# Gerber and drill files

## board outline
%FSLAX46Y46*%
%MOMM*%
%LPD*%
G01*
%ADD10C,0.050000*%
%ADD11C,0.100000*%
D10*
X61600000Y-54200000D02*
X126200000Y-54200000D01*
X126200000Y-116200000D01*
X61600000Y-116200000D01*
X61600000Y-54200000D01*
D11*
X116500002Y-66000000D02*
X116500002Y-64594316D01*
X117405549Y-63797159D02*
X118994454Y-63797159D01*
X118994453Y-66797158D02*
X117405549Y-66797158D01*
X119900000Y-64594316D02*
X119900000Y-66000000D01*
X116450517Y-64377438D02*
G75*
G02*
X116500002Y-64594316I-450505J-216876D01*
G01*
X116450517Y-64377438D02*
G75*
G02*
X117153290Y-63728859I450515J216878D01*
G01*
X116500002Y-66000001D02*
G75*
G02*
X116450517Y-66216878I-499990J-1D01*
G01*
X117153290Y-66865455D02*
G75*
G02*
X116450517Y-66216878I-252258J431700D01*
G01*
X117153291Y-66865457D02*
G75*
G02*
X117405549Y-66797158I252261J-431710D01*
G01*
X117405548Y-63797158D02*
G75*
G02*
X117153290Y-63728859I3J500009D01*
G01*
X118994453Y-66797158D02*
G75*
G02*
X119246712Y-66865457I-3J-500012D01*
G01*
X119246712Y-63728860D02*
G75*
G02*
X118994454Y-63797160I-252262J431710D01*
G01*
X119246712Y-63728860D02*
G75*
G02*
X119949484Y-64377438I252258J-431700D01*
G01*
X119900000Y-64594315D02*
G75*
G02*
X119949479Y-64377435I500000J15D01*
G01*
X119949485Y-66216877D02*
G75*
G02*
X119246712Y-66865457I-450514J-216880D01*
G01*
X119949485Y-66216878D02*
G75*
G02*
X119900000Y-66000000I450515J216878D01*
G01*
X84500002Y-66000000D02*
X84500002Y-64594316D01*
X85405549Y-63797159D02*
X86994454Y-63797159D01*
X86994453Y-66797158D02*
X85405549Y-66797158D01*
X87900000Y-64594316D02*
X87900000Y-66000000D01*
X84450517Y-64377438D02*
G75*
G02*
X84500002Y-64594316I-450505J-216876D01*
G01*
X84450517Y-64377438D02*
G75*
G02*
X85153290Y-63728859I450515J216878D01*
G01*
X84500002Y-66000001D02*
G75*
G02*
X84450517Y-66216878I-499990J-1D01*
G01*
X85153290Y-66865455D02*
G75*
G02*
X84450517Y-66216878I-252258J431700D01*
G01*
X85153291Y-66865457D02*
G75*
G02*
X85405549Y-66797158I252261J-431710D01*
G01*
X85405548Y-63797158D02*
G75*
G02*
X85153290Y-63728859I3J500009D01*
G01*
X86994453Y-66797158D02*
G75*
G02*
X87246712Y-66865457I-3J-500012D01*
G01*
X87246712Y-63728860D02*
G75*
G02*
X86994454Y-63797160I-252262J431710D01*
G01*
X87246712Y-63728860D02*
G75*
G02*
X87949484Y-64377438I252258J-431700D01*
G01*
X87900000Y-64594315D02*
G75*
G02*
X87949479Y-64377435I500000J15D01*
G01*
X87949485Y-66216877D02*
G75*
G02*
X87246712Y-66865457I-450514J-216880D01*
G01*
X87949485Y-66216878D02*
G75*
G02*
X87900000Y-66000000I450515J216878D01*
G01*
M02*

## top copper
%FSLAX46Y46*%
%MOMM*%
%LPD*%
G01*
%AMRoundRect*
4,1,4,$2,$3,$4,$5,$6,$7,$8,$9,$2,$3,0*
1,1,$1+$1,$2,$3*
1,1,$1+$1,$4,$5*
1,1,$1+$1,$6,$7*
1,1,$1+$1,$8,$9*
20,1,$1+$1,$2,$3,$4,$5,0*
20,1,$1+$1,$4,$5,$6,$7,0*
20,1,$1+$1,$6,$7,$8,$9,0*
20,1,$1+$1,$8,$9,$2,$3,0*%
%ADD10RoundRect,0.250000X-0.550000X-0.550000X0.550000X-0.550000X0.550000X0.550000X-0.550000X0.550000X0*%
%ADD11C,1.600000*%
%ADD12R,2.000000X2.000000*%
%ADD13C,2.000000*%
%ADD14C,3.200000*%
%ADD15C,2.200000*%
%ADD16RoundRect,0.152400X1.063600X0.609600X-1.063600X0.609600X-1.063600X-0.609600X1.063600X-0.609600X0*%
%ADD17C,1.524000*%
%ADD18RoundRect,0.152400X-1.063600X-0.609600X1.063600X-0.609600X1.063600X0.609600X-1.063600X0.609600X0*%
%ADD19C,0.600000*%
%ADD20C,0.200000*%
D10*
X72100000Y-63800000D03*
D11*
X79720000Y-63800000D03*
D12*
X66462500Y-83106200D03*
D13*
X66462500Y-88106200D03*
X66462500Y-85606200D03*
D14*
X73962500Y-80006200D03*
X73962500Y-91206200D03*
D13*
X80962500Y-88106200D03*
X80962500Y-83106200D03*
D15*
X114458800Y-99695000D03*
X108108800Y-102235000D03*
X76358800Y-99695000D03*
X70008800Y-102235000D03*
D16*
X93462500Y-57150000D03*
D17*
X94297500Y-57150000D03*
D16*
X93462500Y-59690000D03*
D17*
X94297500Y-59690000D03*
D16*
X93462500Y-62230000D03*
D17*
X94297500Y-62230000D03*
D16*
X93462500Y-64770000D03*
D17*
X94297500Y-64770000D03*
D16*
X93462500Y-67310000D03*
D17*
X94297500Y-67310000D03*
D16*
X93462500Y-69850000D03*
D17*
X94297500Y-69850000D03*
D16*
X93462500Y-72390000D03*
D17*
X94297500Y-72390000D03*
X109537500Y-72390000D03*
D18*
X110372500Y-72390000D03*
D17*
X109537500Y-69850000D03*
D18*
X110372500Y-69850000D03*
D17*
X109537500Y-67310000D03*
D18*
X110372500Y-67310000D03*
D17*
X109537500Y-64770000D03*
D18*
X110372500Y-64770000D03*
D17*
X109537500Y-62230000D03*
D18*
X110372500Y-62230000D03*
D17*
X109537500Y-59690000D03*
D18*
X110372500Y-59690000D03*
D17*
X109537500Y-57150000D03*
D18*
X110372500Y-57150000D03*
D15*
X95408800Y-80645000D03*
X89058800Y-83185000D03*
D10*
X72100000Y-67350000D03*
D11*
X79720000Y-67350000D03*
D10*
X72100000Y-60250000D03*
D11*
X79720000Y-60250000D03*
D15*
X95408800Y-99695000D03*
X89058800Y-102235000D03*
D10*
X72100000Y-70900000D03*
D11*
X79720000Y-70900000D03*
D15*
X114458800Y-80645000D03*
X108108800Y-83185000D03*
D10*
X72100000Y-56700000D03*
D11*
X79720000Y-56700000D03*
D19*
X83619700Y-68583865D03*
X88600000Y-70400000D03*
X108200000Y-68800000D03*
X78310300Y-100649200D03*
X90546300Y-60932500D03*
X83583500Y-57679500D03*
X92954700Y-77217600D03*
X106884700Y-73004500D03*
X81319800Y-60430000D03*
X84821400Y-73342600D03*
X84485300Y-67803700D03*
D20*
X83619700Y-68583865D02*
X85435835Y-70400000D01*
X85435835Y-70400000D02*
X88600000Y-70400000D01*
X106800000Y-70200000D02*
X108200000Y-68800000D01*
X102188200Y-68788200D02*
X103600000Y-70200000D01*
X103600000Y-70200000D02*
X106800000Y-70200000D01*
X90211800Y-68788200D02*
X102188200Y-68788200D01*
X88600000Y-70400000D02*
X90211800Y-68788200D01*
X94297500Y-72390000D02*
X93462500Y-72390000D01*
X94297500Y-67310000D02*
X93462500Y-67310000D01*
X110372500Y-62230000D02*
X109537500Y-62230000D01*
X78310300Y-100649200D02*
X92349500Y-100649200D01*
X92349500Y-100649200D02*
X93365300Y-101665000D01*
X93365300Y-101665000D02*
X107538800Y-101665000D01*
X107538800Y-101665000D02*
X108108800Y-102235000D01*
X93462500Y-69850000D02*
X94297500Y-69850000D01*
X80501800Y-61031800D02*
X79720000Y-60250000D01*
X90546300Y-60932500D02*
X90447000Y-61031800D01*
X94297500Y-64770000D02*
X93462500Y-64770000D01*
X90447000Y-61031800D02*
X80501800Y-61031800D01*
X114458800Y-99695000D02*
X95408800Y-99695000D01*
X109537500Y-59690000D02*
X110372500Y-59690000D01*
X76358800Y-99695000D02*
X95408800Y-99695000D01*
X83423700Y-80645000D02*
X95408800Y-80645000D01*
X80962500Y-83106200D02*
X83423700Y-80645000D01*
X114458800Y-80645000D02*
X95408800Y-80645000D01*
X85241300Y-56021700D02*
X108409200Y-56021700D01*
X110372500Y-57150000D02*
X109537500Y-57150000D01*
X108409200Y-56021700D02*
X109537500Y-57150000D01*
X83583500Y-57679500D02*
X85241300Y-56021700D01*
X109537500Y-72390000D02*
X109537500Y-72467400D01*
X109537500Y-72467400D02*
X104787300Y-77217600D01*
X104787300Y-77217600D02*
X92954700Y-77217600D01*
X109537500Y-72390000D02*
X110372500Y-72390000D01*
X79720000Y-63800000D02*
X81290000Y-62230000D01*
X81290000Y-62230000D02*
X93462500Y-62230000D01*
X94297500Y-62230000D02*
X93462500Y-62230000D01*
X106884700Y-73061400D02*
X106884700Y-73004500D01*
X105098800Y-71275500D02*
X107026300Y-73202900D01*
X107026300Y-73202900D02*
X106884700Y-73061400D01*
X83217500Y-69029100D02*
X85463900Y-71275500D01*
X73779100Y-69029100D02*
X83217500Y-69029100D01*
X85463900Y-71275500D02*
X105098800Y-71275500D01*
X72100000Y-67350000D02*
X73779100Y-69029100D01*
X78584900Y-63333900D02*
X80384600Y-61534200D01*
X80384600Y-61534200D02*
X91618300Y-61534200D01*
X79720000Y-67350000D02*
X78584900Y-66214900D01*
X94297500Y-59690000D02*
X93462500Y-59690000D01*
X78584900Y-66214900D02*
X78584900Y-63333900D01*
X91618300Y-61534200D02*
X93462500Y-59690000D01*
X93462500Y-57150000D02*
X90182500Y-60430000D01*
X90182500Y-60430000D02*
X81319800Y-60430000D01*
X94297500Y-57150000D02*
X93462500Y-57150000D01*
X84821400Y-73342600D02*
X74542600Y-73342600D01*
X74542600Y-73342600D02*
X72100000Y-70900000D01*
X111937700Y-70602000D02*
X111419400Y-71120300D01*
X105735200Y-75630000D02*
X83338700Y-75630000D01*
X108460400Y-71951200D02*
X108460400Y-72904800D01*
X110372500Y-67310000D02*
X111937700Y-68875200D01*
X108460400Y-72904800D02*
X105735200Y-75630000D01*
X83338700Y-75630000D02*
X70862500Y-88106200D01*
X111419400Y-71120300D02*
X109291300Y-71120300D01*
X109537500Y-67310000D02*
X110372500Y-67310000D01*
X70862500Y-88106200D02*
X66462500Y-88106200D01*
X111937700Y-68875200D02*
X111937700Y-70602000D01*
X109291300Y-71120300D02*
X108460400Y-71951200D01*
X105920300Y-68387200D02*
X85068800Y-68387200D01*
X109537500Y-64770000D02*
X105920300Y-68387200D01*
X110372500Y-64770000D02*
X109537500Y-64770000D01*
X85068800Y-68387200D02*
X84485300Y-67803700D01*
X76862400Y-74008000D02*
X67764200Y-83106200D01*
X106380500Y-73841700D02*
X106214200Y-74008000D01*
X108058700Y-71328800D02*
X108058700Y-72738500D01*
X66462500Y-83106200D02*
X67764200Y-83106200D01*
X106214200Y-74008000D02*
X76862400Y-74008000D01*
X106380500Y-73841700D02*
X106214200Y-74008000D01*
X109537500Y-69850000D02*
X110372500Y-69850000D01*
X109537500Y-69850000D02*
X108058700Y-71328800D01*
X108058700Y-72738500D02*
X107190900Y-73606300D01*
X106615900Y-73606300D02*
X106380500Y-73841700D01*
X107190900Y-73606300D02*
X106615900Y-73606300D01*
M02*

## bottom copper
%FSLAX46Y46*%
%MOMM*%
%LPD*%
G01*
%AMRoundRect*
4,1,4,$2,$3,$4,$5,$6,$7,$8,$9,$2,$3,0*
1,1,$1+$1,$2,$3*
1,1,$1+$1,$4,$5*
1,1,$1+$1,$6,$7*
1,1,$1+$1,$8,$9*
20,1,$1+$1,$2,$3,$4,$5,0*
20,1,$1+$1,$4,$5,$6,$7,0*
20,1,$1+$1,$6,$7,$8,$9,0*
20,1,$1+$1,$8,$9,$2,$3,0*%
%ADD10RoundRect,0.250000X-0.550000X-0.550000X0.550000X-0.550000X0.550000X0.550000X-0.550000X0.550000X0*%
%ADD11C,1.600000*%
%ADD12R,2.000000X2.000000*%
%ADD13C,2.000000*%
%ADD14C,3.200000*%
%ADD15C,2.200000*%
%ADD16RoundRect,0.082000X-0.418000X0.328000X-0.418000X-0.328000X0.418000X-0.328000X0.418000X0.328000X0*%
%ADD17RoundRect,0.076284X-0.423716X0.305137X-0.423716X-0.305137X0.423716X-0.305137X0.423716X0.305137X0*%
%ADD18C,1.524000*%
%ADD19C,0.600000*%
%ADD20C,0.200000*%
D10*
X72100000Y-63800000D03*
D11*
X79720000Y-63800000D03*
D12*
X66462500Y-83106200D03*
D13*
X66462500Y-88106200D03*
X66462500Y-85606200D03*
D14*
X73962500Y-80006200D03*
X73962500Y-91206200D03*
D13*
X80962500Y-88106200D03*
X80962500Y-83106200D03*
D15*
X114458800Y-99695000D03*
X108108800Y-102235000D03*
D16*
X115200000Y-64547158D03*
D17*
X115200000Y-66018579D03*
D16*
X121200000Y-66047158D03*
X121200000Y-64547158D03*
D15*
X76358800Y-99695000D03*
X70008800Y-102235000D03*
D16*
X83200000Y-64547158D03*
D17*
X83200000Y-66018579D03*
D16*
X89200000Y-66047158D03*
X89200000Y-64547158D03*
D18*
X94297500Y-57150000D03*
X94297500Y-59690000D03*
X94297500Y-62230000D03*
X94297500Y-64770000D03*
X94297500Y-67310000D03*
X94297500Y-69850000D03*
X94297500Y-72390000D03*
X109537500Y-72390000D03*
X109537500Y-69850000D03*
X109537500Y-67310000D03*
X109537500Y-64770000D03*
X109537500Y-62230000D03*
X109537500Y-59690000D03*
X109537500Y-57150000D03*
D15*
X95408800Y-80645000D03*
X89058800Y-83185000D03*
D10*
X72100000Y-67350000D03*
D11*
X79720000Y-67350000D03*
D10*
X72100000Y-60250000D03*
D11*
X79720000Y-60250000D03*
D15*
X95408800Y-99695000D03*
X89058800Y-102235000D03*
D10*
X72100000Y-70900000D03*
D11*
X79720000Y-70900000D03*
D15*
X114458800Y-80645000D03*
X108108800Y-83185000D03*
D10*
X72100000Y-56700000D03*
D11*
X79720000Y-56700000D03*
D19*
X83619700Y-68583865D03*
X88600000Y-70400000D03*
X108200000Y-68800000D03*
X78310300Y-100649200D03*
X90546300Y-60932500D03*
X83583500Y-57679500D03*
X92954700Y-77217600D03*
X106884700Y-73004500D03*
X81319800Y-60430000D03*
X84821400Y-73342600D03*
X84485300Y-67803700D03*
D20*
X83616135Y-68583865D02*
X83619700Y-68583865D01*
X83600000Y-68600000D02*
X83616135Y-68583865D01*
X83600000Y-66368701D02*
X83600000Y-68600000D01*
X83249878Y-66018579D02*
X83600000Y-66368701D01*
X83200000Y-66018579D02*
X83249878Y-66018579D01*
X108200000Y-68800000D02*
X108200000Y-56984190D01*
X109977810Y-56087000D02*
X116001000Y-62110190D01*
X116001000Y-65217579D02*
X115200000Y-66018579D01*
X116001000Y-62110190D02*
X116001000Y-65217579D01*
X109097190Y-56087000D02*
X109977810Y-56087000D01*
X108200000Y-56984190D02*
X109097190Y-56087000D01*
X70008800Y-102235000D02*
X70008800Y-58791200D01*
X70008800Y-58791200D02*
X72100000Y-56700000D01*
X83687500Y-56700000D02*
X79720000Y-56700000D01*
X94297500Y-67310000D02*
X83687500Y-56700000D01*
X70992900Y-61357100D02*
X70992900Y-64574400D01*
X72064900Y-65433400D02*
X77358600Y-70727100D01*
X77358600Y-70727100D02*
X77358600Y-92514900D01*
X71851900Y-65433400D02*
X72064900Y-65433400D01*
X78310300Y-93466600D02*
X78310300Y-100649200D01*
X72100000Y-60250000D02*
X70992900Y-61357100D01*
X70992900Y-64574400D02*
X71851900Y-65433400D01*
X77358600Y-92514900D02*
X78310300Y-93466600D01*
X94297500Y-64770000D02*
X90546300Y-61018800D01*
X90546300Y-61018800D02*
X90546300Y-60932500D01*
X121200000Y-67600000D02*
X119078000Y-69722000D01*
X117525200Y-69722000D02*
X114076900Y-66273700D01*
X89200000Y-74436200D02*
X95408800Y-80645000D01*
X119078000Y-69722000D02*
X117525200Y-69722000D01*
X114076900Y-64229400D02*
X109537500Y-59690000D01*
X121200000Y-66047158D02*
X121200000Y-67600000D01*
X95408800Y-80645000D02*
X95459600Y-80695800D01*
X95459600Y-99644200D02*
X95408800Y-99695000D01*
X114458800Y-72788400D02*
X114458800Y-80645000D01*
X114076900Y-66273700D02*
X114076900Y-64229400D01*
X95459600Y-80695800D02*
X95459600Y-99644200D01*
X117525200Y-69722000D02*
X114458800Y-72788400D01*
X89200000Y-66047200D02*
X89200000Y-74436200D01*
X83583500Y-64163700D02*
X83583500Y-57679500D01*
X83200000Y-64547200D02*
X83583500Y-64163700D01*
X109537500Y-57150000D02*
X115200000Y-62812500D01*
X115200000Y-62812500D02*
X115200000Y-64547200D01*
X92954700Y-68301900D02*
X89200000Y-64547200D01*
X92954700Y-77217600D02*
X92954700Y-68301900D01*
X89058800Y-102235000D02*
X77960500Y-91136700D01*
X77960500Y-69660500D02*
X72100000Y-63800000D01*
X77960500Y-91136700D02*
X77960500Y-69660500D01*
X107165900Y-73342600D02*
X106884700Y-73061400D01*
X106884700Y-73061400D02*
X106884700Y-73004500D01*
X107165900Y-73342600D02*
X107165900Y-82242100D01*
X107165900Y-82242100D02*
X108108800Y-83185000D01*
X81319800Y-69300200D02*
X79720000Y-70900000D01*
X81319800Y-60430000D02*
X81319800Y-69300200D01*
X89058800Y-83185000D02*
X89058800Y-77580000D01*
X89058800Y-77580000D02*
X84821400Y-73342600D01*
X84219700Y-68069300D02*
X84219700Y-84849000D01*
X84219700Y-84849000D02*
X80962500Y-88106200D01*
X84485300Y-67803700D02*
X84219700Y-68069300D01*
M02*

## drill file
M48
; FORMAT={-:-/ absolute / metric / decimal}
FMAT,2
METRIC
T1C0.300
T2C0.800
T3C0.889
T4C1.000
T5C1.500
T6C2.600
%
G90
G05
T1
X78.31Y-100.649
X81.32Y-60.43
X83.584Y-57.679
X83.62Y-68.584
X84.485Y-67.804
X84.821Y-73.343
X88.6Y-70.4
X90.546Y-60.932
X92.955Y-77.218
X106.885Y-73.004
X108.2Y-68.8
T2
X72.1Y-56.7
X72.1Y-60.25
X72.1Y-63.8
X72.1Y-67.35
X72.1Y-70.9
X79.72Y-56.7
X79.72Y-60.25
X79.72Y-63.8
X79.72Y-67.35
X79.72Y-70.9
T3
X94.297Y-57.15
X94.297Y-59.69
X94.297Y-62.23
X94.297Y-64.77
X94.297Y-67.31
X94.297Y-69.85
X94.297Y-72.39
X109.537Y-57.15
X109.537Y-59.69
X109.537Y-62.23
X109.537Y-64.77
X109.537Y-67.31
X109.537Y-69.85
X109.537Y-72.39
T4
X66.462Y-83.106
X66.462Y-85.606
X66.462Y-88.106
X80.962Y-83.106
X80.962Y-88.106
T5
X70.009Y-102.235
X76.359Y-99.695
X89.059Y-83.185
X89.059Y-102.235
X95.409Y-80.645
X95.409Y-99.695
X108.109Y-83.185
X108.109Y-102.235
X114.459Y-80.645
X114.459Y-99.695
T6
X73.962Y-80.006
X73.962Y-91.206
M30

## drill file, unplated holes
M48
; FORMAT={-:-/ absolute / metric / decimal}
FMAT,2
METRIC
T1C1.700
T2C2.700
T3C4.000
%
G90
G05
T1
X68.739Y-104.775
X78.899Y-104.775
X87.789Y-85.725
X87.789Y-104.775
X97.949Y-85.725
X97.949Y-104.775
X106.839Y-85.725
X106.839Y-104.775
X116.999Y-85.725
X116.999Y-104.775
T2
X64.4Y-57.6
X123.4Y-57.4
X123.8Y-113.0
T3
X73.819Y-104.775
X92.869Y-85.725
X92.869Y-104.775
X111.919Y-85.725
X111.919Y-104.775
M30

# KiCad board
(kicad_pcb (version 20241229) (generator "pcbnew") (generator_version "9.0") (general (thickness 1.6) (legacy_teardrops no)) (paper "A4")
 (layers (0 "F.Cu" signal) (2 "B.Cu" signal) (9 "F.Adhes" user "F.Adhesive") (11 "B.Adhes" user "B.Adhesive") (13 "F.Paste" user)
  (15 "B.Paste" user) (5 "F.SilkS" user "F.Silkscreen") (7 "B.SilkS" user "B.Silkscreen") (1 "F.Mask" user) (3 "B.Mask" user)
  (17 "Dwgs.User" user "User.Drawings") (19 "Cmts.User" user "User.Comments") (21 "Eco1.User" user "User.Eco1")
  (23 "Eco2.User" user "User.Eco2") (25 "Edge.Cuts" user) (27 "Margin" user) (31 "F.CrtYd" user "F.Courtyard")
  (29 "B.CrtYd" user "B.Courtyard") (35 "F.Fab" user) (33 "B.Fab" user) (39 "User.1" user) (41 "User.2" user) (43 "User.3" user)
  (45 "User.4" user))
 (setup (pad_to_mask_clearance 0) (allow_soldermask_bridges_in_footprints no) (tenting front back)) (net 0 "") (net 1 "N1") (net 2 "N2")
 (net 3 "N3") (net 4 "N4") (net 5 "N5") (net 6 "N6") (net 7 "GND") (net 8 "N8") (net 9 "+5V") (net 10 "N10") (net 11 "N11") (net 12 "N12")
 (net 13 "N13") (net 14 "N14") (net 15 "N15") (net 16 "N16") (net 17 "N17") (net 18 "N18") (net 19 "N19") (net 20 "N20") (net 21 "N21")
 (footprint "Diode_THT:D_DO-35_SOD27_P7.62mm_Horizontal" (layer "F.Cu") (at 72.1 63.8)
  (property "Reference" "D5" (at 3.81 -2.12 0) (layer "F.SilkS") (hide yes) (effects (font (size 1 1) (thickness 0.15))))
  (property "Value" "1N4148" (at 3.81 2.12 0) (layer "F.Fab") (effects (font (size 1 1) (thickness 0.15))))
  (pad "1" thru_hole roundrect (at 0 0) (size 1.6 1.6) (drill 0.8) (layers "*.Cu" "*.Mask") (remove_unused_layers no)
   (roundrect_rratio 0.15625) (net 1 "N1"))
  (pad "2" thru_hole circle (at 7.62 0) (size 1.6 1.6) (drill 0.8) (layers "*.Cu" "*.Mask") (remove_unused_layers no) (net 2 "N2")))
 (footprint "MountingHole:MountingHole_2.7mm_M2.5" (layer "F.Cu") (at 123.4 57.4)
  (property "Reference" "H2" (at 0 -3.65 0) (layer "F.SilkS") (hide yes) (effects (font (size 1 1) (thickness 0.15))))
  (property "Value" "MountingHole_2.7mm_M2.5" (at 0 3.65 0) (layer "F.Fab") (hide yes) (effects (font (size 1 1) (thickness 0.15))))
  (pad "" np_thru_hole circle (at 0 0) (size 2.7 2.7) (drill 2.7) (layers "*.Cu" "*.Mask")))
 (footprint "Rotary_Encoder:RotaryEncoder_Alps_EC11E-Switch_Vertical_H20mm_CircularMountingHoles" (layer "F.Cu") (at 66.4625 83.1062)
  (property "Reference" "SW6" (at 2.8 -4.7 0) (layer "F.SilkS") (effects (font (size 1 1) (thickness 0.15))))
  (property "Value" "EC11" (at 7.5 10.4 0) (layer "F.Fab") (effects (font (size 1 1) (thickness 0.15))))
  (pad "A" thru_hole rect (at 0 0) (size 2 2) (drill 1) (layers "*.Cu" "*.Mask") (remove_unused_layers no) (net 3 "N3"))
  (pad "B" thru_hole circle (at 0 5) (size 2 2) (drill 1) (layers "*.Cu" "*.Mask") (remove_unused_layers no) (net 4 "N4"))
  (pad "C" thru_hole circle (at 0 2.5) (size 2 2) (drill 1) (layers "*.Cu" "*.Mask") (remove_unused_layers no) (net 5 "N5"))
  (pad "MP" thru_hole circle (at 7.5 -3.1) (size 3.2 3.2) (drill 2.6) (layers "*.Cu" "*.Mask") (remove_unused_layers no))
  (pad "MP" thru_hole circle (at 7.5 8.1) (size 3.2 3.2) (drill 2.6) (layers "*.Cu" "*.Mask") (remove_unused_layers no))
  (pad "S1" thru_hole circle (at 14.5 5) (size 2 2) (drill 1) (layers "*.Cu" "*.Mask") (remove_unused_layers no) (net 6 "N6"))
  (pad "S2" thru_hole circle (at 14.5 0) (size 2 2) (drill 1) (layers "*.Cu" "*.Mask") (remove_unused_layers no) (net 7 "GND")))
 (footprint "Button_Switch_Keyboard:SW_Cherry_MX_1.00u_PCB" (layer "F.Cu") (at 114.4588 99.695)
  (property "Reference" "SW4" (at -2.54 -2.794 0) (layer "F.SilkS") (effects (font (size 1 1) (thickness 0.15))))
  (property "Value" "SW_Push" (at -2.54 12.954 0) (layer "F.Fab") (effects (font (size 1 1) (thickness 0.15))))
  (pad "" np_thru_hole circle (at -7.62 5.08) (size 1.7 1.7) (drill 1.7) (layers "*.Cu" "*.Mask"))
  (pad "" np_thru_hole circle (at -2.54 5.08) (size 4 4) (drill 4) (layers "*.Cu" "*.Mask"))
  (pad "" np_thru_hole circle (at 2.54 5.08) (size 1.7 1.7) (drill 1.7) (layers "*.Cu" "*.Mask"))
  (pad "1" thru_hole circle (at 0 0) (size 2.2 2.2) (drill 1.5) (layers "*.Cu" "*.Mask") (remove_unused_layers no) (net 7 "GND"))
  (pad "2" thru_hole circle (at -6.35 2.54) (size 2.2 2.2) (drill 1.5) (layers "*.Cu" "*.Mask") (remove_unused_layers no) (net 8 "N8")))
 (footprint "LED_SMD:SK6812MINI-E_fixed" (layer "F.Cu") (at 118.2 65.4)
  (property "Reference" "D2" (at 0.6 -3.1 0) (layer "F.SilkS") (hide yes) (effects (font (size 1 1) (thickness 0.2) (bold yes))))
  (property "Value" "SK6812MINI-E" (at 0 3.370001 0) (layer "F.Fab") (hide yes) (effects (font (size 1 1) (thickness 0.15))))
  (fp_line (start -1.699998 0.6) (end -1.699998 -0.805684) (stroke (width 0.1) (type solid)) (layer "Edge.Cuts"))
  (fp_line (start -0.794451 -1.602841) (end 0.794454 -1.602841) (stroke (width 0.1) (type solid)) (layer "Edge.Cuts"))
  (fp_line (start 0.794453 1.397158) (end -0.794451 1.397158) (stroke (width 0.1) (type solid)) (layer "Edge.Cuts"))
  (fp_line (start 1.7 -0.805684) (end 1.7 0.6) (stroke (width 0.1) (type solid)) (layer "Edge.Cuts"))
  (fp_arc (start -1.749483 -1.022562) (mid -1.712526 -0.91691) (end -1.699998 -0.805684) (stroke (width 0.1) (type solid))
   (layer "Edge.Cuts"))
  (fp_arc (start -1.749483 -1.022562) (mid -1.63807 -1.606877) (end -1.04671 -1.671141) (stroke (width 0.1) (type solid))
   (layer "Edge.Cuts"))
  (fp_arc (start -1.699998 0.600001) (mid -1.712526 0.711226) (end -1.749483 0.816878) (stroke (width 0.1) (type solid)) (layer "Edge.Cuts"))
  (fp_arc (start -1.04671 1.465455) (mid -1.638069 1.401192) (end -1.749483 0.816878) (stroke (width 0.1) (type solid)) (layer "Edge.Cuts"))
  (fp_arc (start -1.046709 1.465457) (mid -0.925121 1.414535) (end -0.794451 1.397158) (stroke (width 0.1) (type solid)) (layer "Edge.Cuts"))
  (fp_arc (start -0.794452 -1.602842) (mid -0.925122 -1.620219) (end -1.04671 -1.671141) (stroke (width 0.1) (type solid))
   (layer "Edge.Cuts"))
  (fp_arc (start 0.794453 1.397158) (mid 0.925124 1.414535) (end 1.046712 1.465457) (stroke (width 0.1) (type solid)) (layer "Edge.Cuts"))
  (fp_arc (start 1.046712 -1.67114) (mid 0.925124 -1.620218) (end 0.794454 -1.602841) (stroke (width 0.1) (type solid)) (layer "Edge.Cuts"))
  (fp_arc (start 1.046712 -1.67114) (mid 1.638072 -1.606876) (end 1.749485 -1.022562) (stroke (width 0.1) (type solid)) (layer "Edge.Cuts"))
  (fp_arc (start 1.7 -0.805685) (mid 1.712528 -0.91691) (end 1.749485 -1.022562) (stroke (width 0.1) (type solid)) (layer "Edge.Cuts"))
  (fp_arc (start 1.749485 0.816877) (mid 1.638073 1.401193) (end 1.046712 1.465457) (stroke (width 0.1) (type solid)) (layer "Edge.Cuts"))
  (fp_arc (start 1.749485 0.816878) (mid 1.712528 0.711226) (end 1.7 0.6) (stroke (width 0.1) (type solid)) (layer "Edge.Cuts"))
  (pad "1" smd roundrect (at -3 -0.852842 270) (size 0.82 1) (layers "B.Cu" "B.Mask" "B.Paste") (roundrect_rratio 0.1) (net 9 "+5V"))
  (pad "2" smd roundrect (at -3 0.618579 270) (size 0.762842 1) (layers "B.Cu" "B.Mask" "B.Paste") (roundrect_rratio 0.1))
  (pad "3" smd roundrect (at 3 0.647158 270) (size 0.82 1) (layers "B.Cu" "B.Mask" "B.Paste") (roundrect_rratio 0.1) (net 7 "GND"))
  (pad "4" smd roundrect (at 3 -0.852842 270) (size 0.82 1) (layers "B.Cu" "B.Mask" "B.Paste") (roundrect_rratio 0.1) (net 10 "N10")))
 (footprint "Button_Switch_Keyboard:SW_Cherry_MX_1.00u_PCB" (layer "F.Cu") (at 76.3588 99.695)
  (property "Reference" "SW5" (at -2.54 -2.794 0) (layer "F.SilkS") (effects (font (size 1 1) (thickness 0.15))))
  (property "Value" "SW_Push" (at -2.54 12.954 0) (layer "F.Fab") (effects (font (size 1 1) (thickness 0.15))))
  (pad "" np_thru_hole circle (at -7.62 5.08) (size 1.7 1.7) (drill 1.7) (layers "*.Cu" "*.Mask"))
  (pad "" np_thru_hole circle (at -2.54 5.08) (size 4 4) (drill 4) (layers "*.Cu" "*.Mask"))
  (pad "" np_thru_hole circle (at 2.54 5.08) (size 1.7 1.7) (drill 1.7) (layers "*.Cu" "*.Mask"))
  (pad "1" thru_hole circle (at 0 0) (size 2.2 2.2) (drill 1.5) (layers "*.Cu" "*.Mask") (remove_unused_layers no) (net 7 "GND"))
  (pad "2" thru_hole circle (at -6.35 2.54) (size 2.2 2.2) (drill 1.5) (layers "*.Cu" "*.Mask") (remove_unused_layers no) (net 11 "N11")))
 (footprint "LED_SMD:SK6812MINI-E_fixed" (layer "F.Cu") (at 86.2 65.4)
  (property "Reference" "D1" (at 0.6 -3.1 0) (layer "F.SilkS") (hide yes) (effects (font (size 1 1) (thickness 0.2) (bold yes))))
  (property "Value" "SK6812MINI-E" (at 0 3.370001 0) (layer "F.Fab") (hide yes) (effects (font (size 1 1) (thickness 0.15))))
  (fp_line (start -1.699998 0.6) (end -1.699998 -0.805684) (stroke (width 0.1) (type solid)) (layer "Edge.Cuts"))
  (fp_line (start -0.794451 -1.602841) (end 0.794454 -1.602841) (stroke (width 0.1) (type solid)) (layer "Edge.Cuts"))
  (fp_line (start 0.794453 1.397158) (end -0.794451 1.397158) (stroke (width 0.1) (type solid)) (layer "Edge.Cuts"))
  (fp_line (start 1.7 -0.805684) (end 1.7 0.6) (stroke (width 0.1) (type solid)) (layer "Edge.Cuts"))
  (fp_arc (start -1.749483 -1.022562) (mid -1.712526 -0.91691) (end -1.699998 -0.805684) (stroke (width 0.1) (type solid))
   (layer "Edge.Cuts"))
  (fp_arc (start -1.749483 -1.022562) (mid -1.63807 -1.606877) (end -1.04671 -1.671141) (stroke (width 0.1) (type solid))
   (layer "Edge.Cuts"))
  (fp_arc (start -1.699998 0.600001) (mid -1.712526 0.711226) (end -1.749483 0.816878) (stroke (width 0.1) (type solid)) (layer "Edge.Cuts"))
  (fp_arc (start -1.04671 1.465455) (mid -1.638069 1.401192) (end -1.749483 0.816878) (stroke (width 0.1) (type solid)) (layer "Edge.Cuts"))
  (fp_arc (start -1.046709 1.465457) (mid -0.925121 1.414535) (end -0.794451 1.397158) (stroke (width 0.1) (type solid)) (layer "Edge.Cuts"))
  (fp_arc (start -0.794452 -1.602842) (mid -0.925122 -1.620219) (end -1.04671 -1.671141) (stroke (width 0.1) (type solid))
   (layer "Edge.Cuts"))
  (fp_arc (start 0.794453 1.397158) (mid 0.925124 1.414535) (end 1.046712 1.465457) (stroke (width 0.1) (type solid)) (layer "Edge.Cuts"))
  (fp_arc (start 1.046712 -1.67114) (mid 0.925124 -1.620218) (end 0.794454 -1.602841) (stroke (width 0.1) (type solid)) (layer "Edge.Cuts"))
  (fp_arc (start 1.046712 -1.67114) (mid 1.638072 -1.606876) (end 1.749485 -1.022562) (stroke (width 0.1) (type solid)) (layer "Edge.Cuts"))
  (fp_arc (start 1.7 -0.805685) (mid 1.712528 -0.91691) (end 1.749485 -1.022562) (stroke (width 0.1) (type solid)) (layer "Edge.Cuts"))
  (fp_arc (start 1.749485 0.816877) (mid 1.638073 1.401193) (end 1.046712 1.465457) (stroke (width 0.1) (type solid)) (layer "Edge.Cuts"))
  (fp_arc (start 1.749485 0.816878) (mid 1.712528 0.711226) (end 1.7 0.6) (stroke (width 0.1) (type solid)) (layer "Edge.Cuts"))
  (pad "1" smd roundrect (at -3 -0.852842 270) (size 0.82 1) (layers "B.Cu" "B.Mask" "B.Paste") (roundrect_rratio 0.1) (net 9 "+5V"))
  (pad "2" smd roundrect (at -3 0.618579 270) (size 0.762842 1) (layers "B.Cu" "B.Mask" "B.Paste") (roundrect_rratio 0.1))
  (pad "3" smd roundrect (at 3 0.647158 270) (size 0.82 1) (layers "B.Cu" "B.Mask" "B.Paste") (roundrect_rratio 0.1) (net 7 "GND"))
  (pad "4" smd roundrect (at 3 -0.852842 270) (size 0.82 1) (layers "B.Cu" "B.Mask" "B.Paste") (roundrect_rratio 0.1) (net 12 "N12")))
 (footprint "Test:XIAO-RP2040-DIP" (layer "F.Cu") (at 101.9175 64.77)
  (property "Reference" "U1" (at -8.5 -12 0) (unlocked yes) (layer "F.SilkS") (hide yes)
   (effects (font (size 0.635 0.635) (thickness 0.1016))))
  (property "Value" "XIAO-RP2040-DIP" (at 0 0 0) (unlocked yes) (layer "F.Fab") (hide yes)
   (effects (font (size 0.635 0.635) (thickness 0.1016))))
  (pad "1" smd roundrect (at -8.455 -7.62 180) (size 2.432 1.524) (layers "F.Cu" "F.Mask") (roundrect_rratio 0.1) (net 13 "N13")
   (thermal_bridge_angle 45))
  (pad "1" thru_hole circle (at -7.62 -7.62 180) (size 1.524 1.524) (drill 0.889) (layers "*.Cu" "*.Mask") (remove_unused_layers no)
   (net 13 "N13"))
  (pad "2" smd roundrect (at -8.455 -5.08 180) (size 2.432 1.524) (layers "F.Cu" "F.Mask") (roundrect_rratio 0.1) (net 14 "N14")
   (thermal_bridge_angle 45))
  (pad "2" thru_hole circle (at -7.62 -5.08 180) (size 1.524 1.524) (drill 0.889) (layers "*.Cu" "*.Mask") (remove_unused_layers no)
   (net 14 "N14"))
  (pad "3" smd roundrect (at -8.455 -2.54 180) (size 2.432 1.524) (layers "F.Cu" "F.Mask") (roundrect_rratio 0.1) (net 2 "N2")
   (thermal_bridge_angle 45))
  (pad "3" thru_hole circle (at -7.62 -2.54 180) (size 1.524 1.524) (drill 0.889) (layers "*.Cu" "*.Mask") (remove_unused_layers no)
   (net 2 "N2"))
  (pad "4" smd roundrect (at -8.455 0 180) (size 2.432 1.524) (layers "F.Cu" "F.Mask") (roundrect_rratio 0.1) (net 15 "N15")
   (thermal_bridge_angle 45))
  (pad "4" thru_hole circle (at -7.62 0 180) (size 1.524 1.524) (drill 0.889) (layers "*.Cu" "*.Mask") (remove_unused_layers no)
   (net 15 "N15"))
  (pad "5" smd roundrect (at -8.455 2.54 180) (size 2.432 1.524) (layers "F.Cu" "F.Mask") (roundrect_rratio 0.1) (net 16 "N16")
   (thermal_bridge_angle 45))
  (pad "5" thru_hole circle (at -7.62 2.54 180) (size 1.524 1.524) (drill 0.889) (layers "*.Cu" "*.Mask") (remove_unused_layers no)
   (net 16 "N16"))
  (pad "6" smd roundrect (at -8.455 5.08 180) (size 2.432 1.524) (layers "F.Cu" "F.Mask") (roundrect_rratio 0.1) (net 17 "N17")
   (thermal_bridge_angle 45))
  (pad "6" thru_hole circle (at -7.62 5.08 180) (size 1.524 1.524) (drill 0.889) (layers "*.Cu" "*.Mask") (remove_unused_layers no)
   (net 17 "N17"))
  (pad "7" smd roundrect (at -8.455 7.62 180) (size 2.432 1.524) (layers "F.Cu" "F.Mask") (roundrect_rratio 0.1) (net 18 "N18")
   (thermal_bridge_angle 45))
  (pad "7" thru_hole circle (at -7.62 7.62 180) (size 1.524 1.524) (drill 0.889) (layers "*.Cu" "*.Mask") (remove_unused_layers no)
   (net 18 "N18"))
  (pad "8" thru_hole circle (at 7.62 7.62) (size 1.524 1.524) (drill 0.889) (layers "*.Cu" "*.Mask") (remove_unused_layers no)
   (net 12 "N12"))
  (pad "8" smd roundrect (at 8.455 7.62) (size 2.432 1.524) (layers "F.Cu" "F.Mask") (roundrect_rratio 0.1) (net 12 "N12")
   (thermal_bridge_angle 45))
  (pad "9" thru_hole circle (at 7.62 5.08) (size 1.524 1.524) (drill 0.889) (layers "*.Cu" "*.Mask") (remove_unused_layers no) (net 3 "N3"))
  (pad "9" smd roundrect (at 8.455 5.08) (size 2.432 1.524) (layers "F.Cu" "F.Mask") (roundrect_rratio 0.1) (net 3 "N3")
   (thermal_bridge_angle 45))
  (pad "10" thru_hole circle (at 7.62 2.54) (size 1.524 1.524) (drill 0.889) (layers "*.Cu" "*.Mask") (remove_unused_layers no) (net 4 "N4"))
  (pad "10" smd roundrect (at 8.455 2.54) (size 2.432 1.524) (layers "F.Cu" "F.Mask") (roundrect_rratio 0.1) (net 4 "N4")
   (thermal_bridge_angle 45))
  (pad "11" thru_hole circle (at 7.62 0) (size 1.524 1.524) (drill 0.889) (layers "*.Cu" "*.Mask") (remove_unused_layers no) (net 6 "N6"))
  (pad "11" smd roundrect (at 8.455 0) (size 2.432 1.524) (layers "F.Cu" "F.Mask") (roundrect_rratio 0.1) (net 6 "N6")
   (thermal_bridge_angle 45))
  (pad "12" thru_hole circle (at 7.62 -2.54) (size 1.524 1.524) (drill 0.889) (layers "*.Cu" "*.Mask") (remove_unused_layers no)
   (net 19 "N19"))
  (pad "12" smd roundrect (at 8.455 -2.54) (size 2.432 1.524) (layers "F.Cu" "F.Mask") (roundrect_rratio 0.1) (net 19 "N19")
   (thermal_bridge_angle 45))
  (pad "13" thru_hole circle (at 7.62 -5.08) (size 1.524 1.524) (drill 0.889) (layers "*.Cu" "*.Mask") (remove_unused_layers no)
   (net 7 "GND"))
  (pad "13" smd roundrect (at 8.455 -5.08) (size 2.432 1.524) (layers "F.Cu" "F.Mask") (roundrect_rratio 0.1) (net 7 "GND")
   (thermal_bridge_angle 45))
  (pad "14" thru_hole circle (at 7.62 -7.62) (size 1.524 1.524) (drill 0.889) (layers "*.Cu" "*.Mask") (remove_unused_layers no)
   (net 9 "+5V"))
  (pad "14" smd roundrect (at 8.455 -7.62) (size 2.432 1.524) (layers "F.Cu" "F.Mask") (roundrect_rratio 0.1) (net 9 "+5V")
   (thermal_bridge_angle 45)))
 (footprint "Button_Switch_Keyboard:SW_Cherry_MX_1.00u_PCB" (layer "F.Cu") (at 95.4088 80.645)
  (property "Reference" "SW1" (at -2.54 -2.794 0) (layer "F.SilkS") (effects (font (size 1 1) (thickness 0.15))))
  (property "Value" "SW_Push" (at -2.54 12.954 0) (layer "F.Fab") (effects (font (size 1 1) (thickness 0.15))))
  (pad "" np_thru_hole circle (at -7.62 5.08) (size 1.7 1.7) (drill 1.7) (layers "*.Cu" "*.Mask"))
  (pad "" np_thru_hole circle (at -2.54 5.08) (size 4 4) (drill 4) (layers "*.Cu" "*.Mask"))
  (pad "" np_thru_hole circle (at 2.54 5.08) (size 1.7 1.7) (drill 1.7) (layers "*.Cu" "*.Mask"))
  (pad "1" thru_hole circle (at 0 0) (size 2.2 2.2) (drill 1.5) (layers "*.Cu" "*.Mask") (remove_unused_layers no) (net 7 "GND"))
  (pad "2" thru_hole circle (at -6.35 2.54) (size 2.2 2.2) (drill 1.5) (layers "*.Cu" "*.Mask") (remove_unused_layers no) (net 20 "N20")))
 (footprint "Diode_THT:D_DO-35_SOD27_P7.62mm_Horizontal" (layer "F.Cu") (at 72.1 67.35)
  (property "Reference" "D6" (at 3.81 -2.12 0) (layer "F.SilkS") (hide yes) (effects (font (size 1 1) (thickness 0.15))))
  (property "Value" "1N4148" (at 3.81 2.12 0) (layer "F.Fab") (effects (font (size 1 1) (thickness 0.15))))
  (pad "1" thru_hole roundrect (at 0 0) (size 1.6 1.6) (drill 0.8) (layers "*.Cu" "*.Mask") (remove_unused_layers no)
   (roundrect_rratio 0.15625) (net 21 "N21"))
  (pad "2" thru_hole circle (at 7.62 0) (size 1.6 1.6) (drill 0.8) (layers "*.Cu" "*.Mask") (remove_unused_layers no) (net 14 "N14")))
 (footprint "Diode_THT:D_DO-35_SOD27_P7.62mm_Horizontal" (layer "F.Cu") (at 72.1 60.25)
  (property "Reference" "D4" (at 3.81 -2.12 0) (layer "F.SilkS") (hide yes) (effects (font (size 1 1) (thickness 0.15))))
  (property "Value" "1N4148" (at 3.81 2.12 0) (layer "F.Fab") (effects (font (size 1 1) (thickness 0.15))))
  (pad "1" thru_hole roundrect (at 0 0) (size 1.6 1.6) (drill 0.8) (layers "*.Cu" "*.Mask") (remove_unused_layers no)
   (roundrect_rratio 0.15625) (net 8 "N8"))
  (pad "2" thru_hole circle (at 7.62 0) (size 1.6 1.6) (drill 0.8) (layers "*.Cu" "*.Mask") (remove_unused_layers no) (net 15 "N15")))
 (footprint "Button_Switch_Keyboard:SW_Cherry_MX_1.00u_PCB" (layer "F.Cu") (at 95.4088 99.695)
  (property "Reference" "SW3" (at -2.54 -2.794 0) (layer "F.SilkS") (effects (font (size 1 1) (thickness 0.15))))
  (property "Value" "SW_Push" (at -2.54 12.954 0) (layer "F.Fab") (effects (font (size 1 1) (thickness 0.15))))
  (pad "" np_thru_hole circle (at -7.62 5.08) (size 1.7 1.7) (drill 1.7) (layers "*.Cu" "*.Mask"))
  (pad "" np_thru_hole circle (at -2.54 5.08) (size 4 4) (drill 4) (layers "*.Cu" "*.Mask"))
  (pad "" np_thru_hole circle (at 2.54 5.08) (size 1.7 1.7) (drill 1.7) (layers "*.Cu" "*.Mask"))
  (pad "1" thru_hole circle (at 0 0) (size 2.2 2.2) (drill 1.5) (layers "*.Cu" "*.Mask") (remove_unused_layers no) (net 7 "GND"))
  (pad "2" thru_hole circle (at -6.35 2.54) (size 2.2 2.2) (drill 1.5) (layers "*.Cu" "*.Mask") (remove_unused_layers no) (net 1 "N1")))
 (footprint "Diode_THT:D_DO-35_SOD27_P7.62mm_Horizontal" (layer "F.Cu") (at 72.1 70.9)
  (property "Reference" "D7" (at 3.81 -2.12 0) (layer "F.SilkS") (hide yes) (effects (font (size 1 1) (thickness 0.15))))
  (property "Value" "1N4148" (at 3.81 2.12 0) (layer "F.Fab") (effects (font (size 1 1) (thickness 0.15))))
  (pad "1" thru_hole roundrect (at 0 0) (size 1.6 1.6) (drill 0.8) (layers "*.Cu" "*.Mask") (remove_unused_layers no)
   (roundrect_rratio 0.15625) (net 20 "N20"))
  (pad "2" thru_hole circle (at 7.62 0) (size 1.6 1.6) (drill 0.8) (layers "*.Cu" "*.Mask") (remove_unused_layers no) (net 13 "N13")))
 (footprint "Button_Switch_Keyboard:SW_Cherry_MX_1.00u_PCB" (layer "F.Cu") (at 114.4588 80.645)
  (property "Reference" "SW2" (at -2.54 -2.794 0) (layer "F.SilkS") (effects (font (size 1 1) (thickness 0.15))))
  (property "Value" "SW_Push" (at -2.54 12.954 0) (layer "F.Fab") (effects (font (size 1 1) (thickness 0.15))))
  (pad "" np_thru_hole circle (at -7.62 5.08) (size 1.7 1.7) (drill 1.7) (layers "*.Cu" "*.Mask"))
  (pad "" np_thru_hole circle (at -2.54 5.08) (size 4 4) (drill 4) (layers "*.Cu" "*.Mask"))
  (pad "" np_thru_hole circle (at 2.54 5.08) (size 1.7 1.7) (drill 1.7) (layers "*.Cu" "*.Mask"))
  (pad "1" thru_hole circle (at 0 0) (size 2.2 2.2) (drill 1.5) (layers "*.Cu" "*.Mask") (remove_unused_layers no) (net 7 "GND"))
  (pad "2" thru_hole circle (at -6.35 2.54) (size 2.2 2.2) (drill 1.5) (layers "*.Cu" "*.Mask") (remove_unused_layers no) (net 21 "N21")))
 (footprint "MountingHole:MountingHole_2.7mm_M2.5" (layer "F.Cu") (at 64.4 57.6)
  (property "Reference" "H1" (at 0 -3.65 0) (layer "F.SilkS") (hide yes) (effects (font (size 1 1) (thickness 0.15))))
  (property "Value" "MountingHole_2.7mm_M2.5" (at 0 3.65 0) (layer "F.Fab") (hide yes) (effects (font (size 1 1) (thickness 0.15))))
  (pad "" np_thru_hole circle (at 0 0) (size 2.7 2.7) (drill 2.7) (layers "*.Cu" "*.Mask")))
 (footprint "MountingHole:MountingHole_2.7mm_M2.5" (layer "F.Cu") (at 123.8 113)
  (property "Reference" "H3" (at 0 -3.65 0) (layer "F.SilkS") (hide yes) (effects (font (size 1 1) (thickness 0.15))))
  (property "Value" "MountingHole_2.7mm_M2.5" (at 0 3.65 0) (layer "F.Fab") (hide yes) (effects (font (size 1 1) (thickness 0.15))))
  (pad "" np_thru_hole circle (at 0 0) (size 2.7 2.7) (drill 2.7) (layers "*.Cu" "*.Mask")))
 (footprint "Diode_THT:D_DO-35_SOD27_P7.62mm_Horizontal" (layer "F.Cu") (at 72.1 56.7)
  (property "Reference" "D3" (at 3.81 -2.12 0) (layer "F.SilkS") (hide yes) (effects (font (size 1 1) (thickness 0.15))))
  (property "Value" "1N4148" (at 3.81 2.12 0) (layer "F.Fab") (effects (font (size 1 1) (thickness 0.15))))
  (pad "1" thru_hole roundrect (at 0 0) (size 1.6 1.6) (drill 0.8) (layers "*.Cu" "*.Mask") (remove_unused_layers no)
   (roundrect_rratio 0.15625) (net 11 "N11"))
  (pad "2" thru_hole circle (at 7.62 0) (size 1.6 1.6) (drill 0.8) (layers "*.Cu" "*.Mask") (remove_unused_layers no) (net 16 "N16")))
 (gr_rect (start 61.6 54.2) (end 126.2 116.2) (stroke (width 0.05) (type default)) (fill no) (layer "Edge.Cuts"))
 (segment (start 85.435835 70.4) (end 88.6 70.4) (width 0.2) (layer "F.Cu") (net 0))
 (segment (start 83.6197 68.583865) (end 85.435835 70.4) (width 0.2) (layer "F.Cu") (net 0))
 (segment (start 106.8 70.2) (end 108.2 68.8) (width 0.2) (layer "F.Cu") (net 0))
 (segment (start 102.1882 68.7882) (end 103.6 70.2) (width 0.2) (layer "F.Cu") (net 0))
 (segment (start 103.6 70.2) (end 106.8 70.2) (width 0.2) (layer "F.Cu") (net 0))
 (segment (start 90.2118 68.7882) (end 102.1882 68.7882) (width 0.2) (layer "F.Cu") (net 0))
 (segment (start 88.6 70.4) (end 90.2118 68.7882) (width 0.2) (layer "F.Cu") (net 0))
 (via (at 83.6197 68.583865) (size 0.6) (drill 0.3) (layers "F.Cu" "B.Cu") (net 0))
 (via (at 88.6 70.4) (size 0.6) (drill 0.3) (layers "F.Cu" "B.Cu") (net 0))
 (via (at 108.2 68.8) (size 0.6) (drill 0.3) (layers "F.Cu" "B.Cu") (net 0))
 (segment (start 83.2 66.018579) (end 83.249878 66.018579) (width 0.2) (layer "B.Cu") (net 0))
 (segment (start 108.2 68.8) (end 108.2 56.98419) (width 0.2) (layer "B.Cu") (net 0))
 (segment (start 109.97781 56.087) (end 116.001 62.11019) (width 0.2) (layer "B.Cu") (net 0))
 (segment (start 83.249878 66.018579) (end 83.6 66.368701) (width 0.2) (layer "B.Cu") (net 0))
 (segment (start 83.616135 68.583865) (end 83.6197 68.583865) (width 0.2) (layer "B.Cu") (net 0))
 (segment (start 116.001 65.217579) (end 115.2 66.018579) (width 0.2) (layer "B.Cu") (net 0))
 (segment (start 116.001 62.11019) (end 116.001 65.217579) (width 0.2) (layer "B.Cu") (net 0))
 (segment (start 83.6 68.6) (end 83.616135 68.583865) (width 0.2) (layer "B.Cu") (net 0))
 (segment (start 109.09719 56.087) (end 109.97781 56.087) (width 0.2) (layer "B.Cu") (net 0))
 (segment (start 83.6 66.368701) (end 83.6 68.6) (width 0.2) (layer "B.Cu") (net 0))
 (segment (start 108.2 56.98419) (end 109.09719 56.087) (width 0.2) (layer "B.Cu") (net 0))
 (segment (start 94.2975 72.39) (end 93.4625 72.39) (width 0.2) (layer "F.Cu") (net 18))
 (segment (start 70.0088 102.235) (end 70.0088 58.7912) (width 0.2) (layer "B.Cu") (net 11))
 (segment (start 70.0088 58.7912) (end 72.1 56.7) (width 0.2) (layer "B.Cu") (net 11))
 (segment (start 94.2975 67.31) (end 93.4625 67.31) (width 0.2) (layer "F.Cu") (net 16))
 (segment (start 83.6875 56.7) (end 79.72 56.7) (width 0.2) (layer "B.Cu") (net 16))
 (segment (start 94.2975 67.31) (end 83.6875 56.7) (width 0.2) (layer "B.Cu") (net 16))
 (segment (start 110.3725 62.23) (end 109.5375 62.23) (width 0.2) (layer "F.Cu") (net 19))
 (segment (start 78.3103 100.6492) (end 92.3495 100.6492) (width 0.2) (layer "F.Cu") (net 8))
 (segment (start 92.3495 100.6492) (end 93.3653 101.665) (width 0.2) (layer "F.Cu") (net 8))
 (segment (start 93.3653 101.665) (end 107.5388 101.665) (width 0.2) (layer "F.Cu") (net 8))
 (segment (start 107.5388 101.665) (end 108.1088 102.235) (width 0.2) (layer "F.Cu") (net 8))
 (via (at 78.3103 100.6492) (size 0.6) (drill 0.3) (layers "F.Cu" "B.Cu") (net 8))
 (segment (start 70.9929 61.3571) (end 70.9929 64.5744) (width 0.2) (layer "B.Cu") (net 8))
 (segment (start 72.0649 65.4334) (end 77.3586 70.7271) (width 0.2) (layer "B.Cu") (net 8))
 (segment (start 77.3586 70.7271) (end 77.3586 92.5149) (width 0.2) (layer "B.Cu") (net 8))
 (segment (start 71.8519 65.4334) (end 72.0649 65.4334) (width 0.2) (layer "B.Cu") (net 8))
 (segment (start 78.3103 93.4666) (end 78.3103 100.6492) (width 0.2) (layer "B.Cu") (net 8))
 (segment (start 72.1 60.25) (end 70.9929 61.3571) (width 0.2) (layer "B.Cu") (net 8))
 (segment (start 70.9929 64.5744) (end 71.8519 65.4334) (width 0.2) (layer "B.Cu") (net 8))
 (segment (start 77.3586 92.5149) (end 78.3103 93.4666) (width 0.2) (layer "B.Cu") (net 8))
 (segment (start 93.4625 69.85) (end 94.2975 69.85) (width 0.2) (layer "F.Cu") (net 17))
 (segment (start 80.5018 61.0318) (end 79.72 60.25) (width 0.2) (layer "F.Cu") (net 15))
 (segment (start 90.5463 60.9325) (end 90.447 61.0318) (width 0.2) (layer "F.Cu") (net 15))
 (segment (start 94.2975 64.77) (end 93.4625 64.77) (width 0.2) (layer "F.Cu") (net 15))
 (segment (start 90.447 61.0318) (end 80.5018 61.0318) (width 0.2) (layer "F.Cu") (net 15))
 (via (at 90.5463 60.9325) (size 0.6) (drill 0.3) (layers "F.Cu" "B.Cu") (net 15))
 (segment (start 94.2975 64.77) (end 90.5463 61.0188) (width 0.2) (layer "B.Cu") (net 15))
 (segment (start 90.5463 61.0188) (end 90.5463 60.9325) (width 0.2) (layer "B.Cu") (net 15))
 (segment (start 114.4588 99.695) (end 95.4088 99.695) (width 0.2) (layer "F.Cu") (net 7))
 (segment (start 109.5375 59.69) (end 110.3725 59.69) (width 0.2) (layer "F.Cu") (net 7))
 (segment (start 76.3588 99.695) (end 95.4088 99.695) (width 0.2) (layer "F.Cu") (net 7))
 (segment (start 83.4237 80.645) (end 95.4088 80.645) (width 0.2) (layer "F.Cu") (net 7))
 (segment (start 80.9625 83.1062) (end 83.4237 80.645) (width 0.2) (layer "F.Cu") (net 7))
 (segment (start 114.4588 80.645) (end 95.4088 80.645) (width 0.2) (layer "F.Cu") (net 7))
 (segment (start 121.2 67.6) (end 119.078 69.722) (width 0.2) (layer "B.Cu") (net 7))
 (segment (start 117.5252 69.722) (end 114.0769 66.2737) (width 0.2) (layer "B.Cu") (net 7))
 (segment (start 89.2 74.4362) (end 95.4088 80.645) (width 0.2) (layer "B.Cu") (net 7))
 (segment (start 119.078 69.722) (end 117.5252 69.722) (width 0.2) (layer "B.Cu") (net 7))
 (segment (start 114.0769 64.2294) (end 109.5375 59.69) (width 0.2) (layer "B.Cu") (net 7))
 (segment (start 121.2 66.047158) (end 121.2 67.6) (width 0.2) (layer "B.Cu") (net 7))
 (segment (start 95.4088 80.645) (end 95.4596 80.6958) (width 0.2) (layer "B.Cu") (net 7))
 (segment (start 95.4596 99.6442) (end 95.4088 99.695) (width 0.2) (layer "B.Cu") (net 7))
 (segment (start 114.4588 72.7884) (end 114.4588 80.645) (width 0.2) (layer "B.Cu") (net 7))
 (segment (start 114.0769 66.2737) (end 114.0769 64.2294) (width 0.2) (layer "B.Cu") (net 7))
 (segment (start 95.4596 80.6958) (end 95.4596 99.6442) (width 0.2) (layer "B.Cu") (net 7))
 (segment (start 117.5252 69.722) (end 114.4588 72.7884) (width 0.2) (layer "B.Cu") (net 7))
 (segment (start 89.2 66.0472) (end 89.2 74.4362) (width 0.2) (layer "B.Cu") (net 7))
 (segment (start 85.2413 56.0217) (end 108.4092 56.0217) (width 0.2) (layer "F.Cu") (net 9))
 (segment (start 110.3725 57.15) (end 109.5375 57.15) (width 0.2) (layer "F.Cu") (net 9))
 (segment (start 108.4092 56.0217) (end 109.5375 57.15) (width 0.2) (layer "F.Cu") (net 9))
 (segment (start 83.5835 57.6795) (end 85.2413 56.0217) (width 0.2) (layer "F.Cu") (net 9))
 (via (at 83.5835 57.6795) (size 0.6) (drill 0.3) (layers "F.Cu" "B.Cu") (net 9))
 (segment (start 83.5835 64.1637) (end 83.5835 57.6795) (width 0.2) (layer "B.Cu") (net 9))
 (segment (start 83.2 64.5472) (end 83.5835 64.1637) (width 0.2) (layer "B.Cu") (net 9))
 (segment (start 109.5375 57.15) (end 115.2 62.8125) (width 0.2) (layer "B.Cu") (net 9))
 (segment (start 115.2 62.8125) (end 115.2 64.5472) (width 0.2) (layer "B.Cu") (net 9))
 (segment (start 109.5375 72.39) (end 109.5375 72.4674) (width 0.2) (layer "F.Cu") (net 12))
 (segment (start 109.5375 72.4674) (end 104.7873 77.2176) (width 0.2) (layer "F.Cu") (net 12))
 (segment (start 104.7873 77.2176) (end 92.9547 77.2176) (width 0.2) (layer "F.Cu") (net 12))
 (segment (start 109.5375 72.39) (end 110.3725 72.39) (width 0.2) (layer "F.Cu") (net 12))
 (via (at 92.9547 77.2176) (size 0.6) (drill 0.3) (layers "F.Cu" "B.Cu") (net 12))
 (segment (start 92.9547 68.3019) (end 89.2 64.5472) (width 0.2) (layer "B.Cu") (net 12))
 (segment (start 92.9547 77.2176) (end 92.9547 68.3019) (width 0.2) (layer "B.Cu") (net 12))
 (segment (start 89.0588 102.235) (end 77.9605 91.1367) (width 0.2) (layer "B.Cu") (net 1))
 (segment (start 77.9605 69.6605) (end 72.1 63.8) (width 0.2) (layer "B.Cu") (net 1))
 (segment (start 77.9605 91.1367) (end 77.9605 69.6605) (width 0.2) (layer "B.Cu") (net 1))
 (segment (start 79.72 63.8) (end 81.29 62.23) (width 0.2) (layer "F.Cu") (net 2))
 (segment (start 81.29 62.23) (end 93.4625 62.23) (width 0.2) (layer "F.Cu") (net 2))
 (segment (start 94.2975 62.23) (end 93.4625 62.23) (width 0.2) (layer "F.Cu") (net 2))
 (segment (start 106.8847 73.0614) (end 106.8847 73.0045) (width 0.2) (layer "F.Cu") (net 21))
 (segment (start 105.0988 71.2755) (end 107.0263 73.2029) (width 0.2) (layer "F.Cu") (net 21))
 (segment (start 107.0263 73.2029) (end 106.8847 73.0614) (width 0.2) (layer "F.Cu") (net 21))
 (segment (start 83.2175 69.0291) (end 85.4639 71.2755) (width 0.2) (layer "F.Cu") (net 21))
 (segment (start 73.7791 69.0291) (end 83.2175 69.0291) (width 0.2) (layer "F.Cu") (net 21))
 (segment (start 85.4639 71.2755) (end 105.0988 71.2755) (width 0.2) (layer "F.Cu") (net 21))
 (segment (start 72.1 67.35) (end 73.7791 69.0291) (width 0.2) (layer "F.Cu") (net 21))
 (via (at 106.8847 73.0045) (size 0.6) (drill 0.3) (layers "F.Cu" "B.Cu") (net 21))
 (segment (start 107.1659 73.3426) (end 106.8847 73.0614) (width 0.2) (layer "B.Cu") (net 21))
 (segment (start 106.8847 73.0614) (end 106.8847 73.0045) (width 0.2) (layer "B.Cu") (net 21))
 (segment (start 107.1659 73.3426) (end 107.1659 82.2421) (width 0.2) (layer "B.Cu") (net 21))
 (segment (start 107.1659 82.2421) (end 108.1088 83.185) (width 0.2) (layer "B.Cu") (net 21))
 (segment (start 78.5849 63.3339) (end 80.3846 61.5342) (width 0.2) (layer "F.Cu") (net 14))
 (segment (start 80.3846 61.5342) (end 91.6183 61.5342) (width 0.2) (layer "F.Cu") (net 14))
 (segment (start 79.72 67.35) (end 78.5849 66.2149) (width 0.2) (layer "F.Cu") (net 14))
 (segment (start 94.2975 59.69) (end 93.4625 59.69) (width 0.2) (layer "F.Cu") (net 14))
 (segment (start 78.5849 66.2149) (end 78.5849 63.3339) (width 0.2) (layer "F.Cu") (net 14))
 (segment (start 91.6183 61.5342) (end 93.4625 59.69) (width 0.2) (layer "F.Cu") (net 14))
 (segment (start 93.4625 57.15) (end 90.1825 60.43) (width 0.2) (layer "F.Cu") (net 13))
 (segment (start 90.1825 60.43) (end 81.3198 60.43) (width 0.2) (layer "F.Cu") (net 13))
 (segment (start 94.2975 57.15) (end 93.4625 57.15) (width 0.2) (layer "F.Cu") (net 13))
 (via (at 81.3198 60.43) (size 0.6) (drill 0.3) (layers "F.Cu" "B.Cu") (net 13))
 (segment (start 81.3198 69.3002) (end 79.72 70.9) (width 0.2) (layer "B.Cu") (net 13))
 (segment (start 81.3198 60.43) (end 81.3198 69.3002) (width 0.2) (layer "B.Cu") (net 13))
 (segment (start 84.8214 73.3426) (end 74.5426 73.3426) (width 0.2) (layer "F.Cu") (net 20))
 (segment (start 74.5426 73.3426) (end 72.1 70.9) (width 0.2) (layer "F.Cu") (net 20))
 (via (at 84.8214 73.3426) (size 0.6) (drill 0.3) (layers "F.Cu" "B.Cu") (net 20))
 (segment (start 89.0588 83.185) (end 89.0588 77.58) (width 0.2) (layer "B.Cu") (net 20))
 (segment (start 89.0588 77.58) (end 84.8214 73.3426) (width 0.2) (layer "B.Cu") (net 20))
 (segment (start 111.9377 70.602) (end 111.4194 71.1203) (width 0.2) (layer "F.Cu") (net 4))
 (segment (start 105.7352 75.63) (end 83.3387 75.63) (width 0.2) (layer "F.Cu") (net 4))
 (segment (start 108.4604 71.9512) (end 108.4604 72.9048) (width 0.2) (layer "F.Cu") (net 4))
 (segment (start 110.3725 67.31) (end 111.9377 68.8752) (width 0.2) (layer "F.Cu") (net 4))
 (segment (start 108.4604 72.9048) (end 105.7352 75.63) (width 0.2) (layer "F.Cu") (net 4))
 (segment (start 83.3387 75.63) (end 70.8625 88.1062) (width 0.2) (layer "F.Cu") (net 4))
 (segment (start 111.4194 71.1203) (end 109.2913 71.1203) (width 0.2) (layer "F.Cu") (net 4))
 (segment (start 109.5375 67.31) (end 110.3725 67.31) (width 0.2) (layer "F.Cu") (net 4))
 (segment (start 70.8625 88.1062) (end 66.4625 88.1062) (width 0.2) (layer "F.Cu") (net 4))
 (segment (start 111.9377 68.8752) (end 111.9377 70.602) (width 0.2) (layer "F.Cu") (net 4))
 (segment (start 109.2913 71.1203) (end 108.4604 71.9512) (width 0.2) (layer "F.Cu") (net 4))
 (segment (start 105.9203 68.3872) (end 85.0688 68.3872) (width 0.2) (layer "F.Cu") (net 6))
 (segment (start 109.5375 64.77) (end 105.9203 68.3872) (width 0.2) (layer "F.Cu") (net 6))
 (segment (start 110.3725 64.77) (end 109.5375 64.77) (width 0.2) (layer "F.Cu") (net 6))
 (segment (start 85.0688 68.3872) (end 84.4853 67.8037) (width 0.2) (layer "F.Cu") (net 6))
 (via (at 84.4853 67.8037) (size 0.6) (drill 0.3) (layers "F.Cu" "B.Cu") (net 6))
 (segment (start 84.2197 68.0693) (end 84.2197 84.849) (width 0.2) (layer "B.Cu") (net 6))
 (segment (start 84.2197 84.849) (end 80.9625 88.1062) (width 0.2) (layer "B.Cu") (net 6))
 (segment (start 84.4853 67.8037) (end 84.2197 68.0693) (width 0.2) (layer "B.Cu") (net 6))
 (segment (start 76.8624 74.008) (end 67.7642 83.1062) (width 0.2) (layer "F.Cu") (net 3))
 (segment (start 106.3805 73.8417) (end 106.2142 74.008) (width 0.2) (layer "F.Cu") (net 3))
 (segment (start 108.0587 71.3288) (end 108.0587 72.7385) (width 0.2) (layer "F.Cu") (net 3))
 (segment (start 66.4625 83.1062) (end 67.7642 83.1062) (width 0.2) (layer "F.Cu") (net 3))
 (segment (start 106.2142 74.008) (end 76.8624 74.008) (width 0.2) (layer "F.Cu") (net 3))
 (segment (start 106.3805 73.8417) (end 106.2142 74.008) (width 0.2) (layer "F.Cu") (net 3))
 (segment (start 109.5375 69.85) (end 110.3725 69.85) (width 0.2) (layer "F.Cu") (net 3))
 (segment (start 109.5375 69.85) (end 108.0587 71.3288) (width 0.2) (layer "F.Cu") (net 3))
 (segment (start 108.0587 72.7385) (end 107.1909 73.6063) (width 0.2) (layer "F.Cu") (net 3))
 (segment (start 106.6159 73.6063) (end 106.3805 73.8417) (width 0.2) (layer "F.Cu") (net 3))
 (segment (start 107.1909 73.6063) (end 106.6159 73.6063) (width 0.2) (layer "F.Cu") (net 3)))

